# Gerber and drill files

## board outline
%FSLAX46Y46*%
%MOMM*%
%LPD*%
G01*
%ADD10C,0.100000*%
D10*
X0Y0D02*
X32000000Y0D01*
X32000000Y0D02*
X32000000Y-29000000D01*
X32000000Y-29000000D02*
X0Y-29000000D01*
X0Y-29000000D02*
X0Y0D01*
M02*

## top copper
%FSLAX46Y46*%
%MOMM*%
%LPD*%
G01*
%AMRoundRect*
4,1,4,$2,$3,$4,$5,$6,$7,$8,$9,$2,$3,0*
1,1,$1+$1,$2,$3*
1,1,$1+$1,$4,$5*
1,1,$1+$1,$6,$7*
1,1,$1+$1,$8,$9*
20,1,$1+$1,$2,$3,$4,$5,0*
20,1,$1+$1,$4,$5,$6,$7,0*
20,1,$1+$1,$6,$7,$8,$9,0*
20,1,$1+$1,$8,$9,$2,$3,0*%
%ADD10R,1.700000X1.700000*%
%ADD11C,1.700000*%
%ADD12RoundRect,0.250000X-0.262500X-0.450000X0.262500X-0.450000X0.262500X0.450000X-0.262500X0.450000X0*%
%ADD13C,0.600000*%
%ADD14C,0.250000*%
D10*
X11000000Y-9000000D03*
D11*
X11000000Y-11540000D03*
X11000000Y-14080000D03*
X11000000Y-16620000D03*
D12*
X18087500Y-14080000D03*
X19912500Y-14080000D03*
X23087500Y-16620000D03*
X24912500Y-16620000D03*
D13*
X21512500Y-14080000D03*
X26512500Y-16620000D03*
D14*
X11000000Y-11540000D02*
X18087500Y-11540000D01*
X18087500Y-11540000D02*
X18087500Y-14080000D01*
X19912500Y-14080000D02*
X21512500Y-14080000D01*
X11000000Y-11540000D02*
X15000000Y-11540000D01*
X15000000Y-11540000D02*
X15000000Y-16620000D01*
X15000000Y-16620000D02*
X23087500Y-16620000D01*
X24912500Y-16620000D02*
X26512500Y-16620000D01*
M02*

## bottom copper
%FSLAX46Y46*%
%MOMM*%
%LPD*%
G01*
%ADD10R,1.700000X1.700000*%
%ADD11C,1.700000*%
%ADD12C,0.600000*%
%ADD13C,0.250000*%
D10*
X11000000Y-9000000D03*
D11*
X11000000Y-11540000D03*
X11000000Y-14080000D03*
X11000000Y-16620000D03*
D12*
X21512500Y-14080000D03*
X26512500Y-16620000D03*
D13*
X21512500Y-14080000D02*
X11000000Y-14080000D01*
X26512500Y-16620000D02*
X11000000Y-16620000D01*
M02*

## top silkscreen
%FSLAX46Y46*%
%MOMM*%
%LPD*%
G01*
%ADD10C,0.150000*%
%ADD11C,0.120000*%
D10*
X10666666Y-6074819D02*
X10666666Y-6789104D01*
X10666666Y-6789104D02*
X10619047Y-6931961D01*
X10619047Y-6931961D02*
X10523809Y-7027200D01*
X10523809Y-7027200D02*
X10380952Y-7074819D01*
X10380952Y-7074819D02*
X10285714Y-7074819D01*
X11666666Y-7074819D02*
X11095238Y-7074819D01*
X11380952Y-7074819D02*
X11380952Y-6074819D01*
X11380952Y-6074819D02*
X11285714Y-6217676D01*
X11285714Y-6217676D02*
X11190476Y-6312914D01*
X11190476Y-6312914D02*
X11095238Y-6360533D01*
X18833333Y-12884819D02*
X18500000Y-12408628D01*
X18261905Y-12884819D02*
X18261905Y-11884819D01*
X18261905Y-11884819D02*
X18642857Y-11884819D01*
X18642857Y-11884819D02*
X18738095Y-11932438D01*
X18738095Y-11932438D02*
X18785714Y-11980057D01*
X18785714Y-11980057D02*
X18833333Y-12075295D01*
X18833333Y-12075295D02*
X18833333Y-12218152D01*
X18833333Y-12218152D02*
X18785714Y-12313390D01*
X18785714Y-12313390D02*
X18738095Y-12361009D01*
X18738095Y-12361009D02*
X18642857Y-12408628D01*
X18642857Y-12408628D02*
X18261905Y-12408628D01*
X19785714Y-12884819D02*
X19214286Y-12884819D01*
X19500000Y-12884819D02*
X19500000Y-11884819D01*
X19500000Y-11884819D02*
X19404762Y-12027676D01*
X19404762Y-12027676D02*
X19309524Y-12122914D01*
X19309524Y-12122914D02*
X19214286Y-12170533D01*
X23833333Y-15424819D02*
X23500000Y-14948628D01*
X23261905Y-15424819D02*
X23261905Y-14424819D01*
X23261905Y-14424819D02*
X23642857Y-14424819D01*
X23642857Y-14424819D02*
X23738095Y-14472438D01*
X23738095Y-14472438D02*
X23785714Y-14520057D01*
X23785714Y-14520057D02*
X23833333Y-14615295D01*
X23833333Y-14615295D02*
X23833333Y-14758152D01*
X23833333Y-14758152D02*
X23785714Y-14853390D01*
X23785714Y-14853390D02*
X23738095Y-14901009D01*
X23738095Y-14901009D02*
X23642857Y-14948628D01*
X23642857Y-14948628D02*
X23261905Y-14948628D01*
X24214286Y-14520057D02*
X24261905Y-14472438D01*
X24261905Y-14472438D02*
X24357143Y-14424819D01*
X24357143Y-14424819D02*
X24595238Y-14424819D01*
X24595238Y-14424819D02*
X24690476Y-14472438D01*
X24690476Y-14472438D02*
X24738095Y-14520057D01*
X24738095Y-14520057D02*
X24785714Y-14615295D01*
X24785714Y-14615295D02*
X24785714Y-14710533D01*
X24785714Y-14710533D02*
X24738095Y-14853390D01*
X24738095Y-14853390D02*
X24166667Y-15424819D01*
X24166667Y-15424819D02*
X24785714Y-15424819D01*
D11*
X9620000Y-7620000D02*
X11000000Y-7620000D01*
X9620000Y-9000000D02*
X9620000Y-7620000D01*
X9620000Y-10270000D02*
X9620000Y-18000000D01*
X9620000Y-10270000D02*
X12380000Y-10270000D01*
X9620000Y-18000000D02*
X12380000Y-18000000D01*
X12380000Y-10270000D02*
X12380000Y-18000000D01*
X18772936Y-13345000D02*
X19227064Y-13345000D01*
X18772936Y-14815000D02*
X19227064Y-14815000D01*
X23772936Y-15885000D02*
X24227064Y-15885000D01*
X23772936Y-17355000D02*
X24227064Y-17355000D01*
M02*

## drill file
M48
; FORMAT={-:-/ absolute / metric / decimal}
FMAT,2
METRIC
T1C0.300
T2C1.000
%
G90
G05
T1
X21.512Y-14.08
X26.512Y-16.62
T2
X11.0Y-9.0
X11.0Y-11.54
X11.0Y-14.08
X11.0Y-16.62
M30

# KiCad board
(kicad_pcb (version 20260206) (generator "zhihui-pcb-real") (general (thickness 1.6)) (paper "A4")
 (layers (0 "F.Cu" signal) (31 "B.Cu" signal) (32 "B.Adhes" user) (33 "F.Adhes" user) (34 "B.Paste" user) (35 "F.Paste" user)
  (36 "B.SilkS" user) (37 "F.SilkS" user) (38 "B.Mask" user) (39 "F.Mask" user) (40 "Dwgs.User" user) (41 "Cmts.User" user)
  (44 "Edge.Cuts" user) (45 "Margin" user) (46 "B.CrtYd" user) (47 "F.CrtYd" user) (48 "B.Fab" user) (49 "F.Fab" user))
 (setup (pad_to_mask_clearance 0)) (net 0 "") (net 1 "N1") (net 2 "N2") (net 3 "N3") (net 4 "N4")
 (gr_line (start 0 0) (end 32 0) (stroke (width 0.1) (type default)) (layer "Edge.Cuts"))
 (gr_line (start 32 0) (end 32 29) (stroke (width 0.1) (type default)) (layer "Edge.Cuts"))
 (gr_line (start 32 29) (end 0 29) (stroke (width 0.1) (type default)) (layer "Edge.Cuts"))
 (gr_line (start 0 29) (end 0 0) (stroke (width 0.1) (type default)) (layer "Edge.Cuts"))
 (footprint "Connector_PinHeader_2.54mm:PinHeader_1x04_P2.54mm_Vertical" (layer "F.Cu")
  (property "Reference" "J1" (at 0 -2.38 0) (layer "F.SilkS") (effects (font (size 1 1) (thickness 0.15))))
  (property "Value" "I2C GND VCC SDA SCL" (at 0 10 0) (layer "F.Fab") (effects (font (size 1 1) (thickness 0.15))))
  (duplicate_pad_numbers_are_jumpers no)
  (fp_line (start -1.38 -1.38) (end 0 -1.38) (stroke (width 0.12) (type solid)) (layer "F.SilkS"))
  (fp_line (start -1.38 0) (end -1.38 -1.38) (stroke (width 0.12) (type solid)) (layer "F.SilkS"))
  (fp_line (start -1.38 1.27) (end -1.38 9) (stroke (width 0.12) (type solid)) (layer "F.SilkS"))
  (fp_line (start -1.38 1.27) (end 1.38 1.27) (stroke (width 0.12) (type solid)) (layer "F.SilkS"))
  (fp_line (start -1.38 9) (end 1.38 9) (stroke (width 0.12) (type solid)) (layer "F.SilkS"))
  (fp_line (start 1.38 1.27) (end 1.38 9) (stroke (width 0.12) (type solid)) (layer "F.SilkS"))
  (pad "1" thru_hole rect (at 0 0) (size 1.7 1.7) (drill 1) (layers "*.Cu" "*.Mask") (remove_unused_layers no) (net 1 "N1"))
  (pad "2" thru_hole circle (at 0 2.54) (size 1.7 1.7) (drill 1) (layers "*.Cu" "*.Mask") (remove_unused_layers no) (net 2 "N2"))
  (pad "3" thru_hole circle (at 0 5.08) (size 1.7 1.7) (drill 1) (layers "*.Cu" "*.Mask") (remove_unused_layers no) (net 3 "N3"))
  (pad "4" thru_hole circle (at 0 7.62) (size 1.7 1.7) (drill 1) (layers "*.Cu" "*.Mask") (remove_unused_layers no) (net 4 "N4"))
  (at 11 9 0))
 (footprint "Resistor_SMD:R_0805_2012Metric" (layer "F.Cu")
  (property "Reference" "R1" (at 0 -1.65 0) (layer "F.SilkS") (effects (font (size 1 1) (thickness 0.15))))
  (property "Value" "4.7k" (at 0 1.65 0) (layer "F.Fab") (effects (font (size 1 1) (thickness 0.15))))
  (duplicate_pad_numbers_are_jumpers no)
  (fp_line (start -0.227064 -0.735) (end 0.227064 -0.735) (stroke (width 0.12) (type solid)) (layer "F.SilkS"))
  (fp_line (start -0.227064 0.735) (end 0.227064 0.735) (stroke (width 0.12) (type solid)) (layer "F.SilkS"))
  (pad "1" smd roundrect (at -0.9125 0) (size 1.025 1.4) (layers "F.Cu" "F.Mask" "F.Paste") (roundrect_rratio 0.243902) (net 2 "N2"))
  (pad "2" smd roundrect (at 0.9125 0) (size 1.025 1.4) (layers "F.Cu" "F.Mask" "F.Paste") (roundrect_rratio 0.243902) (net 3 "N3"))
  (at 19 14.08 0))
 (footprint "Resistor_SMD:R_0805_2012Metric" (layer "F.Cu")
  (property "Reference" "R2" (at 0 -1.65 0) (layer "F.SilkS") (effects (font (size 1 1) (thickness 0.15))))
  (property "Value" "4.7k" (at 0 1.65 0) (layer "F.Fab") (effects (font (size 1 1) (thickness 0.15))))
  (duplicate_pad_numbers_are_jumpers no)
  (fp_line (start -0.227064 -0.735) (end 0.227064 -0.735) (stroke (width 0.12) (type solid)) (layer "F.SilkS"))
  (fp_line (start -0.227064 0.735) (end 0.227064 0.735) (stroke (width 0.12) (type solid)) (layer "F.SilkS"))
  (pad "1" smd roundrect (at -0.9125 0) (size 1.025 1.4) (layers "F.Cu" "F.Mask" "F.Paste") (roundrect_rratio 0.243902) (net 2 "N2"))
  (pad "2" smd roundrect (at 0.9125 0) (size 1.025 1.4) (layers "F.Cu" "F.Mask" "F.Paste") (roundrect_rratio 0.243902) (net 4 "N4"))
  (at 24 16.62 0))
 (segment (start 11 11.54) (end 18.0875 11.54) (width 0.25) (layer "F.Cu") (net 2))
 (segment (start 18.0875 11.54) (end 18.0875 14.08) (width 0.25) (layer "F.Cu") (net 2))
 (segment (start 19.9125 14.08) (end 21.5125 14.08) (width 0.25) (layer "F.Cu") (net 3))
 (segment (start 21.5125 14.08) (end 11 14.08) (width 0.25) (layer "B.Cu") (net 3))
 (segment (start 11 11.54) (end 15 11.54) (width 0.25) (layer "F.Cu") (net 2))
 (segment (start 15 11.54) (end 15 16.62) (width 0.25) (layer "F.Cu") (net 2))
 (segment (start 15 16.62) (end 23.0875 16.62) (width 0.25) (layer "F.Cu") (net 2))
 (segment (start 24.9125 16.62) (end 26.5125 16.62) (width 0.25) (layer "F.Cu") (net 4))
 (segment (start 26.5125 16.62) (end 11 16.62) (width 0.25) (layer "B.Cu") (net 4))
 (via (at 21.5125 14.08) (size 0.6) (drill 0.3) (layers "F.Cu" "B.Cu") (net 3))
 (via (at 26.5125 16.62) (size 0.6) (drill 0.3) (layers "F.Cu" "B.Cu") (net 4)))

